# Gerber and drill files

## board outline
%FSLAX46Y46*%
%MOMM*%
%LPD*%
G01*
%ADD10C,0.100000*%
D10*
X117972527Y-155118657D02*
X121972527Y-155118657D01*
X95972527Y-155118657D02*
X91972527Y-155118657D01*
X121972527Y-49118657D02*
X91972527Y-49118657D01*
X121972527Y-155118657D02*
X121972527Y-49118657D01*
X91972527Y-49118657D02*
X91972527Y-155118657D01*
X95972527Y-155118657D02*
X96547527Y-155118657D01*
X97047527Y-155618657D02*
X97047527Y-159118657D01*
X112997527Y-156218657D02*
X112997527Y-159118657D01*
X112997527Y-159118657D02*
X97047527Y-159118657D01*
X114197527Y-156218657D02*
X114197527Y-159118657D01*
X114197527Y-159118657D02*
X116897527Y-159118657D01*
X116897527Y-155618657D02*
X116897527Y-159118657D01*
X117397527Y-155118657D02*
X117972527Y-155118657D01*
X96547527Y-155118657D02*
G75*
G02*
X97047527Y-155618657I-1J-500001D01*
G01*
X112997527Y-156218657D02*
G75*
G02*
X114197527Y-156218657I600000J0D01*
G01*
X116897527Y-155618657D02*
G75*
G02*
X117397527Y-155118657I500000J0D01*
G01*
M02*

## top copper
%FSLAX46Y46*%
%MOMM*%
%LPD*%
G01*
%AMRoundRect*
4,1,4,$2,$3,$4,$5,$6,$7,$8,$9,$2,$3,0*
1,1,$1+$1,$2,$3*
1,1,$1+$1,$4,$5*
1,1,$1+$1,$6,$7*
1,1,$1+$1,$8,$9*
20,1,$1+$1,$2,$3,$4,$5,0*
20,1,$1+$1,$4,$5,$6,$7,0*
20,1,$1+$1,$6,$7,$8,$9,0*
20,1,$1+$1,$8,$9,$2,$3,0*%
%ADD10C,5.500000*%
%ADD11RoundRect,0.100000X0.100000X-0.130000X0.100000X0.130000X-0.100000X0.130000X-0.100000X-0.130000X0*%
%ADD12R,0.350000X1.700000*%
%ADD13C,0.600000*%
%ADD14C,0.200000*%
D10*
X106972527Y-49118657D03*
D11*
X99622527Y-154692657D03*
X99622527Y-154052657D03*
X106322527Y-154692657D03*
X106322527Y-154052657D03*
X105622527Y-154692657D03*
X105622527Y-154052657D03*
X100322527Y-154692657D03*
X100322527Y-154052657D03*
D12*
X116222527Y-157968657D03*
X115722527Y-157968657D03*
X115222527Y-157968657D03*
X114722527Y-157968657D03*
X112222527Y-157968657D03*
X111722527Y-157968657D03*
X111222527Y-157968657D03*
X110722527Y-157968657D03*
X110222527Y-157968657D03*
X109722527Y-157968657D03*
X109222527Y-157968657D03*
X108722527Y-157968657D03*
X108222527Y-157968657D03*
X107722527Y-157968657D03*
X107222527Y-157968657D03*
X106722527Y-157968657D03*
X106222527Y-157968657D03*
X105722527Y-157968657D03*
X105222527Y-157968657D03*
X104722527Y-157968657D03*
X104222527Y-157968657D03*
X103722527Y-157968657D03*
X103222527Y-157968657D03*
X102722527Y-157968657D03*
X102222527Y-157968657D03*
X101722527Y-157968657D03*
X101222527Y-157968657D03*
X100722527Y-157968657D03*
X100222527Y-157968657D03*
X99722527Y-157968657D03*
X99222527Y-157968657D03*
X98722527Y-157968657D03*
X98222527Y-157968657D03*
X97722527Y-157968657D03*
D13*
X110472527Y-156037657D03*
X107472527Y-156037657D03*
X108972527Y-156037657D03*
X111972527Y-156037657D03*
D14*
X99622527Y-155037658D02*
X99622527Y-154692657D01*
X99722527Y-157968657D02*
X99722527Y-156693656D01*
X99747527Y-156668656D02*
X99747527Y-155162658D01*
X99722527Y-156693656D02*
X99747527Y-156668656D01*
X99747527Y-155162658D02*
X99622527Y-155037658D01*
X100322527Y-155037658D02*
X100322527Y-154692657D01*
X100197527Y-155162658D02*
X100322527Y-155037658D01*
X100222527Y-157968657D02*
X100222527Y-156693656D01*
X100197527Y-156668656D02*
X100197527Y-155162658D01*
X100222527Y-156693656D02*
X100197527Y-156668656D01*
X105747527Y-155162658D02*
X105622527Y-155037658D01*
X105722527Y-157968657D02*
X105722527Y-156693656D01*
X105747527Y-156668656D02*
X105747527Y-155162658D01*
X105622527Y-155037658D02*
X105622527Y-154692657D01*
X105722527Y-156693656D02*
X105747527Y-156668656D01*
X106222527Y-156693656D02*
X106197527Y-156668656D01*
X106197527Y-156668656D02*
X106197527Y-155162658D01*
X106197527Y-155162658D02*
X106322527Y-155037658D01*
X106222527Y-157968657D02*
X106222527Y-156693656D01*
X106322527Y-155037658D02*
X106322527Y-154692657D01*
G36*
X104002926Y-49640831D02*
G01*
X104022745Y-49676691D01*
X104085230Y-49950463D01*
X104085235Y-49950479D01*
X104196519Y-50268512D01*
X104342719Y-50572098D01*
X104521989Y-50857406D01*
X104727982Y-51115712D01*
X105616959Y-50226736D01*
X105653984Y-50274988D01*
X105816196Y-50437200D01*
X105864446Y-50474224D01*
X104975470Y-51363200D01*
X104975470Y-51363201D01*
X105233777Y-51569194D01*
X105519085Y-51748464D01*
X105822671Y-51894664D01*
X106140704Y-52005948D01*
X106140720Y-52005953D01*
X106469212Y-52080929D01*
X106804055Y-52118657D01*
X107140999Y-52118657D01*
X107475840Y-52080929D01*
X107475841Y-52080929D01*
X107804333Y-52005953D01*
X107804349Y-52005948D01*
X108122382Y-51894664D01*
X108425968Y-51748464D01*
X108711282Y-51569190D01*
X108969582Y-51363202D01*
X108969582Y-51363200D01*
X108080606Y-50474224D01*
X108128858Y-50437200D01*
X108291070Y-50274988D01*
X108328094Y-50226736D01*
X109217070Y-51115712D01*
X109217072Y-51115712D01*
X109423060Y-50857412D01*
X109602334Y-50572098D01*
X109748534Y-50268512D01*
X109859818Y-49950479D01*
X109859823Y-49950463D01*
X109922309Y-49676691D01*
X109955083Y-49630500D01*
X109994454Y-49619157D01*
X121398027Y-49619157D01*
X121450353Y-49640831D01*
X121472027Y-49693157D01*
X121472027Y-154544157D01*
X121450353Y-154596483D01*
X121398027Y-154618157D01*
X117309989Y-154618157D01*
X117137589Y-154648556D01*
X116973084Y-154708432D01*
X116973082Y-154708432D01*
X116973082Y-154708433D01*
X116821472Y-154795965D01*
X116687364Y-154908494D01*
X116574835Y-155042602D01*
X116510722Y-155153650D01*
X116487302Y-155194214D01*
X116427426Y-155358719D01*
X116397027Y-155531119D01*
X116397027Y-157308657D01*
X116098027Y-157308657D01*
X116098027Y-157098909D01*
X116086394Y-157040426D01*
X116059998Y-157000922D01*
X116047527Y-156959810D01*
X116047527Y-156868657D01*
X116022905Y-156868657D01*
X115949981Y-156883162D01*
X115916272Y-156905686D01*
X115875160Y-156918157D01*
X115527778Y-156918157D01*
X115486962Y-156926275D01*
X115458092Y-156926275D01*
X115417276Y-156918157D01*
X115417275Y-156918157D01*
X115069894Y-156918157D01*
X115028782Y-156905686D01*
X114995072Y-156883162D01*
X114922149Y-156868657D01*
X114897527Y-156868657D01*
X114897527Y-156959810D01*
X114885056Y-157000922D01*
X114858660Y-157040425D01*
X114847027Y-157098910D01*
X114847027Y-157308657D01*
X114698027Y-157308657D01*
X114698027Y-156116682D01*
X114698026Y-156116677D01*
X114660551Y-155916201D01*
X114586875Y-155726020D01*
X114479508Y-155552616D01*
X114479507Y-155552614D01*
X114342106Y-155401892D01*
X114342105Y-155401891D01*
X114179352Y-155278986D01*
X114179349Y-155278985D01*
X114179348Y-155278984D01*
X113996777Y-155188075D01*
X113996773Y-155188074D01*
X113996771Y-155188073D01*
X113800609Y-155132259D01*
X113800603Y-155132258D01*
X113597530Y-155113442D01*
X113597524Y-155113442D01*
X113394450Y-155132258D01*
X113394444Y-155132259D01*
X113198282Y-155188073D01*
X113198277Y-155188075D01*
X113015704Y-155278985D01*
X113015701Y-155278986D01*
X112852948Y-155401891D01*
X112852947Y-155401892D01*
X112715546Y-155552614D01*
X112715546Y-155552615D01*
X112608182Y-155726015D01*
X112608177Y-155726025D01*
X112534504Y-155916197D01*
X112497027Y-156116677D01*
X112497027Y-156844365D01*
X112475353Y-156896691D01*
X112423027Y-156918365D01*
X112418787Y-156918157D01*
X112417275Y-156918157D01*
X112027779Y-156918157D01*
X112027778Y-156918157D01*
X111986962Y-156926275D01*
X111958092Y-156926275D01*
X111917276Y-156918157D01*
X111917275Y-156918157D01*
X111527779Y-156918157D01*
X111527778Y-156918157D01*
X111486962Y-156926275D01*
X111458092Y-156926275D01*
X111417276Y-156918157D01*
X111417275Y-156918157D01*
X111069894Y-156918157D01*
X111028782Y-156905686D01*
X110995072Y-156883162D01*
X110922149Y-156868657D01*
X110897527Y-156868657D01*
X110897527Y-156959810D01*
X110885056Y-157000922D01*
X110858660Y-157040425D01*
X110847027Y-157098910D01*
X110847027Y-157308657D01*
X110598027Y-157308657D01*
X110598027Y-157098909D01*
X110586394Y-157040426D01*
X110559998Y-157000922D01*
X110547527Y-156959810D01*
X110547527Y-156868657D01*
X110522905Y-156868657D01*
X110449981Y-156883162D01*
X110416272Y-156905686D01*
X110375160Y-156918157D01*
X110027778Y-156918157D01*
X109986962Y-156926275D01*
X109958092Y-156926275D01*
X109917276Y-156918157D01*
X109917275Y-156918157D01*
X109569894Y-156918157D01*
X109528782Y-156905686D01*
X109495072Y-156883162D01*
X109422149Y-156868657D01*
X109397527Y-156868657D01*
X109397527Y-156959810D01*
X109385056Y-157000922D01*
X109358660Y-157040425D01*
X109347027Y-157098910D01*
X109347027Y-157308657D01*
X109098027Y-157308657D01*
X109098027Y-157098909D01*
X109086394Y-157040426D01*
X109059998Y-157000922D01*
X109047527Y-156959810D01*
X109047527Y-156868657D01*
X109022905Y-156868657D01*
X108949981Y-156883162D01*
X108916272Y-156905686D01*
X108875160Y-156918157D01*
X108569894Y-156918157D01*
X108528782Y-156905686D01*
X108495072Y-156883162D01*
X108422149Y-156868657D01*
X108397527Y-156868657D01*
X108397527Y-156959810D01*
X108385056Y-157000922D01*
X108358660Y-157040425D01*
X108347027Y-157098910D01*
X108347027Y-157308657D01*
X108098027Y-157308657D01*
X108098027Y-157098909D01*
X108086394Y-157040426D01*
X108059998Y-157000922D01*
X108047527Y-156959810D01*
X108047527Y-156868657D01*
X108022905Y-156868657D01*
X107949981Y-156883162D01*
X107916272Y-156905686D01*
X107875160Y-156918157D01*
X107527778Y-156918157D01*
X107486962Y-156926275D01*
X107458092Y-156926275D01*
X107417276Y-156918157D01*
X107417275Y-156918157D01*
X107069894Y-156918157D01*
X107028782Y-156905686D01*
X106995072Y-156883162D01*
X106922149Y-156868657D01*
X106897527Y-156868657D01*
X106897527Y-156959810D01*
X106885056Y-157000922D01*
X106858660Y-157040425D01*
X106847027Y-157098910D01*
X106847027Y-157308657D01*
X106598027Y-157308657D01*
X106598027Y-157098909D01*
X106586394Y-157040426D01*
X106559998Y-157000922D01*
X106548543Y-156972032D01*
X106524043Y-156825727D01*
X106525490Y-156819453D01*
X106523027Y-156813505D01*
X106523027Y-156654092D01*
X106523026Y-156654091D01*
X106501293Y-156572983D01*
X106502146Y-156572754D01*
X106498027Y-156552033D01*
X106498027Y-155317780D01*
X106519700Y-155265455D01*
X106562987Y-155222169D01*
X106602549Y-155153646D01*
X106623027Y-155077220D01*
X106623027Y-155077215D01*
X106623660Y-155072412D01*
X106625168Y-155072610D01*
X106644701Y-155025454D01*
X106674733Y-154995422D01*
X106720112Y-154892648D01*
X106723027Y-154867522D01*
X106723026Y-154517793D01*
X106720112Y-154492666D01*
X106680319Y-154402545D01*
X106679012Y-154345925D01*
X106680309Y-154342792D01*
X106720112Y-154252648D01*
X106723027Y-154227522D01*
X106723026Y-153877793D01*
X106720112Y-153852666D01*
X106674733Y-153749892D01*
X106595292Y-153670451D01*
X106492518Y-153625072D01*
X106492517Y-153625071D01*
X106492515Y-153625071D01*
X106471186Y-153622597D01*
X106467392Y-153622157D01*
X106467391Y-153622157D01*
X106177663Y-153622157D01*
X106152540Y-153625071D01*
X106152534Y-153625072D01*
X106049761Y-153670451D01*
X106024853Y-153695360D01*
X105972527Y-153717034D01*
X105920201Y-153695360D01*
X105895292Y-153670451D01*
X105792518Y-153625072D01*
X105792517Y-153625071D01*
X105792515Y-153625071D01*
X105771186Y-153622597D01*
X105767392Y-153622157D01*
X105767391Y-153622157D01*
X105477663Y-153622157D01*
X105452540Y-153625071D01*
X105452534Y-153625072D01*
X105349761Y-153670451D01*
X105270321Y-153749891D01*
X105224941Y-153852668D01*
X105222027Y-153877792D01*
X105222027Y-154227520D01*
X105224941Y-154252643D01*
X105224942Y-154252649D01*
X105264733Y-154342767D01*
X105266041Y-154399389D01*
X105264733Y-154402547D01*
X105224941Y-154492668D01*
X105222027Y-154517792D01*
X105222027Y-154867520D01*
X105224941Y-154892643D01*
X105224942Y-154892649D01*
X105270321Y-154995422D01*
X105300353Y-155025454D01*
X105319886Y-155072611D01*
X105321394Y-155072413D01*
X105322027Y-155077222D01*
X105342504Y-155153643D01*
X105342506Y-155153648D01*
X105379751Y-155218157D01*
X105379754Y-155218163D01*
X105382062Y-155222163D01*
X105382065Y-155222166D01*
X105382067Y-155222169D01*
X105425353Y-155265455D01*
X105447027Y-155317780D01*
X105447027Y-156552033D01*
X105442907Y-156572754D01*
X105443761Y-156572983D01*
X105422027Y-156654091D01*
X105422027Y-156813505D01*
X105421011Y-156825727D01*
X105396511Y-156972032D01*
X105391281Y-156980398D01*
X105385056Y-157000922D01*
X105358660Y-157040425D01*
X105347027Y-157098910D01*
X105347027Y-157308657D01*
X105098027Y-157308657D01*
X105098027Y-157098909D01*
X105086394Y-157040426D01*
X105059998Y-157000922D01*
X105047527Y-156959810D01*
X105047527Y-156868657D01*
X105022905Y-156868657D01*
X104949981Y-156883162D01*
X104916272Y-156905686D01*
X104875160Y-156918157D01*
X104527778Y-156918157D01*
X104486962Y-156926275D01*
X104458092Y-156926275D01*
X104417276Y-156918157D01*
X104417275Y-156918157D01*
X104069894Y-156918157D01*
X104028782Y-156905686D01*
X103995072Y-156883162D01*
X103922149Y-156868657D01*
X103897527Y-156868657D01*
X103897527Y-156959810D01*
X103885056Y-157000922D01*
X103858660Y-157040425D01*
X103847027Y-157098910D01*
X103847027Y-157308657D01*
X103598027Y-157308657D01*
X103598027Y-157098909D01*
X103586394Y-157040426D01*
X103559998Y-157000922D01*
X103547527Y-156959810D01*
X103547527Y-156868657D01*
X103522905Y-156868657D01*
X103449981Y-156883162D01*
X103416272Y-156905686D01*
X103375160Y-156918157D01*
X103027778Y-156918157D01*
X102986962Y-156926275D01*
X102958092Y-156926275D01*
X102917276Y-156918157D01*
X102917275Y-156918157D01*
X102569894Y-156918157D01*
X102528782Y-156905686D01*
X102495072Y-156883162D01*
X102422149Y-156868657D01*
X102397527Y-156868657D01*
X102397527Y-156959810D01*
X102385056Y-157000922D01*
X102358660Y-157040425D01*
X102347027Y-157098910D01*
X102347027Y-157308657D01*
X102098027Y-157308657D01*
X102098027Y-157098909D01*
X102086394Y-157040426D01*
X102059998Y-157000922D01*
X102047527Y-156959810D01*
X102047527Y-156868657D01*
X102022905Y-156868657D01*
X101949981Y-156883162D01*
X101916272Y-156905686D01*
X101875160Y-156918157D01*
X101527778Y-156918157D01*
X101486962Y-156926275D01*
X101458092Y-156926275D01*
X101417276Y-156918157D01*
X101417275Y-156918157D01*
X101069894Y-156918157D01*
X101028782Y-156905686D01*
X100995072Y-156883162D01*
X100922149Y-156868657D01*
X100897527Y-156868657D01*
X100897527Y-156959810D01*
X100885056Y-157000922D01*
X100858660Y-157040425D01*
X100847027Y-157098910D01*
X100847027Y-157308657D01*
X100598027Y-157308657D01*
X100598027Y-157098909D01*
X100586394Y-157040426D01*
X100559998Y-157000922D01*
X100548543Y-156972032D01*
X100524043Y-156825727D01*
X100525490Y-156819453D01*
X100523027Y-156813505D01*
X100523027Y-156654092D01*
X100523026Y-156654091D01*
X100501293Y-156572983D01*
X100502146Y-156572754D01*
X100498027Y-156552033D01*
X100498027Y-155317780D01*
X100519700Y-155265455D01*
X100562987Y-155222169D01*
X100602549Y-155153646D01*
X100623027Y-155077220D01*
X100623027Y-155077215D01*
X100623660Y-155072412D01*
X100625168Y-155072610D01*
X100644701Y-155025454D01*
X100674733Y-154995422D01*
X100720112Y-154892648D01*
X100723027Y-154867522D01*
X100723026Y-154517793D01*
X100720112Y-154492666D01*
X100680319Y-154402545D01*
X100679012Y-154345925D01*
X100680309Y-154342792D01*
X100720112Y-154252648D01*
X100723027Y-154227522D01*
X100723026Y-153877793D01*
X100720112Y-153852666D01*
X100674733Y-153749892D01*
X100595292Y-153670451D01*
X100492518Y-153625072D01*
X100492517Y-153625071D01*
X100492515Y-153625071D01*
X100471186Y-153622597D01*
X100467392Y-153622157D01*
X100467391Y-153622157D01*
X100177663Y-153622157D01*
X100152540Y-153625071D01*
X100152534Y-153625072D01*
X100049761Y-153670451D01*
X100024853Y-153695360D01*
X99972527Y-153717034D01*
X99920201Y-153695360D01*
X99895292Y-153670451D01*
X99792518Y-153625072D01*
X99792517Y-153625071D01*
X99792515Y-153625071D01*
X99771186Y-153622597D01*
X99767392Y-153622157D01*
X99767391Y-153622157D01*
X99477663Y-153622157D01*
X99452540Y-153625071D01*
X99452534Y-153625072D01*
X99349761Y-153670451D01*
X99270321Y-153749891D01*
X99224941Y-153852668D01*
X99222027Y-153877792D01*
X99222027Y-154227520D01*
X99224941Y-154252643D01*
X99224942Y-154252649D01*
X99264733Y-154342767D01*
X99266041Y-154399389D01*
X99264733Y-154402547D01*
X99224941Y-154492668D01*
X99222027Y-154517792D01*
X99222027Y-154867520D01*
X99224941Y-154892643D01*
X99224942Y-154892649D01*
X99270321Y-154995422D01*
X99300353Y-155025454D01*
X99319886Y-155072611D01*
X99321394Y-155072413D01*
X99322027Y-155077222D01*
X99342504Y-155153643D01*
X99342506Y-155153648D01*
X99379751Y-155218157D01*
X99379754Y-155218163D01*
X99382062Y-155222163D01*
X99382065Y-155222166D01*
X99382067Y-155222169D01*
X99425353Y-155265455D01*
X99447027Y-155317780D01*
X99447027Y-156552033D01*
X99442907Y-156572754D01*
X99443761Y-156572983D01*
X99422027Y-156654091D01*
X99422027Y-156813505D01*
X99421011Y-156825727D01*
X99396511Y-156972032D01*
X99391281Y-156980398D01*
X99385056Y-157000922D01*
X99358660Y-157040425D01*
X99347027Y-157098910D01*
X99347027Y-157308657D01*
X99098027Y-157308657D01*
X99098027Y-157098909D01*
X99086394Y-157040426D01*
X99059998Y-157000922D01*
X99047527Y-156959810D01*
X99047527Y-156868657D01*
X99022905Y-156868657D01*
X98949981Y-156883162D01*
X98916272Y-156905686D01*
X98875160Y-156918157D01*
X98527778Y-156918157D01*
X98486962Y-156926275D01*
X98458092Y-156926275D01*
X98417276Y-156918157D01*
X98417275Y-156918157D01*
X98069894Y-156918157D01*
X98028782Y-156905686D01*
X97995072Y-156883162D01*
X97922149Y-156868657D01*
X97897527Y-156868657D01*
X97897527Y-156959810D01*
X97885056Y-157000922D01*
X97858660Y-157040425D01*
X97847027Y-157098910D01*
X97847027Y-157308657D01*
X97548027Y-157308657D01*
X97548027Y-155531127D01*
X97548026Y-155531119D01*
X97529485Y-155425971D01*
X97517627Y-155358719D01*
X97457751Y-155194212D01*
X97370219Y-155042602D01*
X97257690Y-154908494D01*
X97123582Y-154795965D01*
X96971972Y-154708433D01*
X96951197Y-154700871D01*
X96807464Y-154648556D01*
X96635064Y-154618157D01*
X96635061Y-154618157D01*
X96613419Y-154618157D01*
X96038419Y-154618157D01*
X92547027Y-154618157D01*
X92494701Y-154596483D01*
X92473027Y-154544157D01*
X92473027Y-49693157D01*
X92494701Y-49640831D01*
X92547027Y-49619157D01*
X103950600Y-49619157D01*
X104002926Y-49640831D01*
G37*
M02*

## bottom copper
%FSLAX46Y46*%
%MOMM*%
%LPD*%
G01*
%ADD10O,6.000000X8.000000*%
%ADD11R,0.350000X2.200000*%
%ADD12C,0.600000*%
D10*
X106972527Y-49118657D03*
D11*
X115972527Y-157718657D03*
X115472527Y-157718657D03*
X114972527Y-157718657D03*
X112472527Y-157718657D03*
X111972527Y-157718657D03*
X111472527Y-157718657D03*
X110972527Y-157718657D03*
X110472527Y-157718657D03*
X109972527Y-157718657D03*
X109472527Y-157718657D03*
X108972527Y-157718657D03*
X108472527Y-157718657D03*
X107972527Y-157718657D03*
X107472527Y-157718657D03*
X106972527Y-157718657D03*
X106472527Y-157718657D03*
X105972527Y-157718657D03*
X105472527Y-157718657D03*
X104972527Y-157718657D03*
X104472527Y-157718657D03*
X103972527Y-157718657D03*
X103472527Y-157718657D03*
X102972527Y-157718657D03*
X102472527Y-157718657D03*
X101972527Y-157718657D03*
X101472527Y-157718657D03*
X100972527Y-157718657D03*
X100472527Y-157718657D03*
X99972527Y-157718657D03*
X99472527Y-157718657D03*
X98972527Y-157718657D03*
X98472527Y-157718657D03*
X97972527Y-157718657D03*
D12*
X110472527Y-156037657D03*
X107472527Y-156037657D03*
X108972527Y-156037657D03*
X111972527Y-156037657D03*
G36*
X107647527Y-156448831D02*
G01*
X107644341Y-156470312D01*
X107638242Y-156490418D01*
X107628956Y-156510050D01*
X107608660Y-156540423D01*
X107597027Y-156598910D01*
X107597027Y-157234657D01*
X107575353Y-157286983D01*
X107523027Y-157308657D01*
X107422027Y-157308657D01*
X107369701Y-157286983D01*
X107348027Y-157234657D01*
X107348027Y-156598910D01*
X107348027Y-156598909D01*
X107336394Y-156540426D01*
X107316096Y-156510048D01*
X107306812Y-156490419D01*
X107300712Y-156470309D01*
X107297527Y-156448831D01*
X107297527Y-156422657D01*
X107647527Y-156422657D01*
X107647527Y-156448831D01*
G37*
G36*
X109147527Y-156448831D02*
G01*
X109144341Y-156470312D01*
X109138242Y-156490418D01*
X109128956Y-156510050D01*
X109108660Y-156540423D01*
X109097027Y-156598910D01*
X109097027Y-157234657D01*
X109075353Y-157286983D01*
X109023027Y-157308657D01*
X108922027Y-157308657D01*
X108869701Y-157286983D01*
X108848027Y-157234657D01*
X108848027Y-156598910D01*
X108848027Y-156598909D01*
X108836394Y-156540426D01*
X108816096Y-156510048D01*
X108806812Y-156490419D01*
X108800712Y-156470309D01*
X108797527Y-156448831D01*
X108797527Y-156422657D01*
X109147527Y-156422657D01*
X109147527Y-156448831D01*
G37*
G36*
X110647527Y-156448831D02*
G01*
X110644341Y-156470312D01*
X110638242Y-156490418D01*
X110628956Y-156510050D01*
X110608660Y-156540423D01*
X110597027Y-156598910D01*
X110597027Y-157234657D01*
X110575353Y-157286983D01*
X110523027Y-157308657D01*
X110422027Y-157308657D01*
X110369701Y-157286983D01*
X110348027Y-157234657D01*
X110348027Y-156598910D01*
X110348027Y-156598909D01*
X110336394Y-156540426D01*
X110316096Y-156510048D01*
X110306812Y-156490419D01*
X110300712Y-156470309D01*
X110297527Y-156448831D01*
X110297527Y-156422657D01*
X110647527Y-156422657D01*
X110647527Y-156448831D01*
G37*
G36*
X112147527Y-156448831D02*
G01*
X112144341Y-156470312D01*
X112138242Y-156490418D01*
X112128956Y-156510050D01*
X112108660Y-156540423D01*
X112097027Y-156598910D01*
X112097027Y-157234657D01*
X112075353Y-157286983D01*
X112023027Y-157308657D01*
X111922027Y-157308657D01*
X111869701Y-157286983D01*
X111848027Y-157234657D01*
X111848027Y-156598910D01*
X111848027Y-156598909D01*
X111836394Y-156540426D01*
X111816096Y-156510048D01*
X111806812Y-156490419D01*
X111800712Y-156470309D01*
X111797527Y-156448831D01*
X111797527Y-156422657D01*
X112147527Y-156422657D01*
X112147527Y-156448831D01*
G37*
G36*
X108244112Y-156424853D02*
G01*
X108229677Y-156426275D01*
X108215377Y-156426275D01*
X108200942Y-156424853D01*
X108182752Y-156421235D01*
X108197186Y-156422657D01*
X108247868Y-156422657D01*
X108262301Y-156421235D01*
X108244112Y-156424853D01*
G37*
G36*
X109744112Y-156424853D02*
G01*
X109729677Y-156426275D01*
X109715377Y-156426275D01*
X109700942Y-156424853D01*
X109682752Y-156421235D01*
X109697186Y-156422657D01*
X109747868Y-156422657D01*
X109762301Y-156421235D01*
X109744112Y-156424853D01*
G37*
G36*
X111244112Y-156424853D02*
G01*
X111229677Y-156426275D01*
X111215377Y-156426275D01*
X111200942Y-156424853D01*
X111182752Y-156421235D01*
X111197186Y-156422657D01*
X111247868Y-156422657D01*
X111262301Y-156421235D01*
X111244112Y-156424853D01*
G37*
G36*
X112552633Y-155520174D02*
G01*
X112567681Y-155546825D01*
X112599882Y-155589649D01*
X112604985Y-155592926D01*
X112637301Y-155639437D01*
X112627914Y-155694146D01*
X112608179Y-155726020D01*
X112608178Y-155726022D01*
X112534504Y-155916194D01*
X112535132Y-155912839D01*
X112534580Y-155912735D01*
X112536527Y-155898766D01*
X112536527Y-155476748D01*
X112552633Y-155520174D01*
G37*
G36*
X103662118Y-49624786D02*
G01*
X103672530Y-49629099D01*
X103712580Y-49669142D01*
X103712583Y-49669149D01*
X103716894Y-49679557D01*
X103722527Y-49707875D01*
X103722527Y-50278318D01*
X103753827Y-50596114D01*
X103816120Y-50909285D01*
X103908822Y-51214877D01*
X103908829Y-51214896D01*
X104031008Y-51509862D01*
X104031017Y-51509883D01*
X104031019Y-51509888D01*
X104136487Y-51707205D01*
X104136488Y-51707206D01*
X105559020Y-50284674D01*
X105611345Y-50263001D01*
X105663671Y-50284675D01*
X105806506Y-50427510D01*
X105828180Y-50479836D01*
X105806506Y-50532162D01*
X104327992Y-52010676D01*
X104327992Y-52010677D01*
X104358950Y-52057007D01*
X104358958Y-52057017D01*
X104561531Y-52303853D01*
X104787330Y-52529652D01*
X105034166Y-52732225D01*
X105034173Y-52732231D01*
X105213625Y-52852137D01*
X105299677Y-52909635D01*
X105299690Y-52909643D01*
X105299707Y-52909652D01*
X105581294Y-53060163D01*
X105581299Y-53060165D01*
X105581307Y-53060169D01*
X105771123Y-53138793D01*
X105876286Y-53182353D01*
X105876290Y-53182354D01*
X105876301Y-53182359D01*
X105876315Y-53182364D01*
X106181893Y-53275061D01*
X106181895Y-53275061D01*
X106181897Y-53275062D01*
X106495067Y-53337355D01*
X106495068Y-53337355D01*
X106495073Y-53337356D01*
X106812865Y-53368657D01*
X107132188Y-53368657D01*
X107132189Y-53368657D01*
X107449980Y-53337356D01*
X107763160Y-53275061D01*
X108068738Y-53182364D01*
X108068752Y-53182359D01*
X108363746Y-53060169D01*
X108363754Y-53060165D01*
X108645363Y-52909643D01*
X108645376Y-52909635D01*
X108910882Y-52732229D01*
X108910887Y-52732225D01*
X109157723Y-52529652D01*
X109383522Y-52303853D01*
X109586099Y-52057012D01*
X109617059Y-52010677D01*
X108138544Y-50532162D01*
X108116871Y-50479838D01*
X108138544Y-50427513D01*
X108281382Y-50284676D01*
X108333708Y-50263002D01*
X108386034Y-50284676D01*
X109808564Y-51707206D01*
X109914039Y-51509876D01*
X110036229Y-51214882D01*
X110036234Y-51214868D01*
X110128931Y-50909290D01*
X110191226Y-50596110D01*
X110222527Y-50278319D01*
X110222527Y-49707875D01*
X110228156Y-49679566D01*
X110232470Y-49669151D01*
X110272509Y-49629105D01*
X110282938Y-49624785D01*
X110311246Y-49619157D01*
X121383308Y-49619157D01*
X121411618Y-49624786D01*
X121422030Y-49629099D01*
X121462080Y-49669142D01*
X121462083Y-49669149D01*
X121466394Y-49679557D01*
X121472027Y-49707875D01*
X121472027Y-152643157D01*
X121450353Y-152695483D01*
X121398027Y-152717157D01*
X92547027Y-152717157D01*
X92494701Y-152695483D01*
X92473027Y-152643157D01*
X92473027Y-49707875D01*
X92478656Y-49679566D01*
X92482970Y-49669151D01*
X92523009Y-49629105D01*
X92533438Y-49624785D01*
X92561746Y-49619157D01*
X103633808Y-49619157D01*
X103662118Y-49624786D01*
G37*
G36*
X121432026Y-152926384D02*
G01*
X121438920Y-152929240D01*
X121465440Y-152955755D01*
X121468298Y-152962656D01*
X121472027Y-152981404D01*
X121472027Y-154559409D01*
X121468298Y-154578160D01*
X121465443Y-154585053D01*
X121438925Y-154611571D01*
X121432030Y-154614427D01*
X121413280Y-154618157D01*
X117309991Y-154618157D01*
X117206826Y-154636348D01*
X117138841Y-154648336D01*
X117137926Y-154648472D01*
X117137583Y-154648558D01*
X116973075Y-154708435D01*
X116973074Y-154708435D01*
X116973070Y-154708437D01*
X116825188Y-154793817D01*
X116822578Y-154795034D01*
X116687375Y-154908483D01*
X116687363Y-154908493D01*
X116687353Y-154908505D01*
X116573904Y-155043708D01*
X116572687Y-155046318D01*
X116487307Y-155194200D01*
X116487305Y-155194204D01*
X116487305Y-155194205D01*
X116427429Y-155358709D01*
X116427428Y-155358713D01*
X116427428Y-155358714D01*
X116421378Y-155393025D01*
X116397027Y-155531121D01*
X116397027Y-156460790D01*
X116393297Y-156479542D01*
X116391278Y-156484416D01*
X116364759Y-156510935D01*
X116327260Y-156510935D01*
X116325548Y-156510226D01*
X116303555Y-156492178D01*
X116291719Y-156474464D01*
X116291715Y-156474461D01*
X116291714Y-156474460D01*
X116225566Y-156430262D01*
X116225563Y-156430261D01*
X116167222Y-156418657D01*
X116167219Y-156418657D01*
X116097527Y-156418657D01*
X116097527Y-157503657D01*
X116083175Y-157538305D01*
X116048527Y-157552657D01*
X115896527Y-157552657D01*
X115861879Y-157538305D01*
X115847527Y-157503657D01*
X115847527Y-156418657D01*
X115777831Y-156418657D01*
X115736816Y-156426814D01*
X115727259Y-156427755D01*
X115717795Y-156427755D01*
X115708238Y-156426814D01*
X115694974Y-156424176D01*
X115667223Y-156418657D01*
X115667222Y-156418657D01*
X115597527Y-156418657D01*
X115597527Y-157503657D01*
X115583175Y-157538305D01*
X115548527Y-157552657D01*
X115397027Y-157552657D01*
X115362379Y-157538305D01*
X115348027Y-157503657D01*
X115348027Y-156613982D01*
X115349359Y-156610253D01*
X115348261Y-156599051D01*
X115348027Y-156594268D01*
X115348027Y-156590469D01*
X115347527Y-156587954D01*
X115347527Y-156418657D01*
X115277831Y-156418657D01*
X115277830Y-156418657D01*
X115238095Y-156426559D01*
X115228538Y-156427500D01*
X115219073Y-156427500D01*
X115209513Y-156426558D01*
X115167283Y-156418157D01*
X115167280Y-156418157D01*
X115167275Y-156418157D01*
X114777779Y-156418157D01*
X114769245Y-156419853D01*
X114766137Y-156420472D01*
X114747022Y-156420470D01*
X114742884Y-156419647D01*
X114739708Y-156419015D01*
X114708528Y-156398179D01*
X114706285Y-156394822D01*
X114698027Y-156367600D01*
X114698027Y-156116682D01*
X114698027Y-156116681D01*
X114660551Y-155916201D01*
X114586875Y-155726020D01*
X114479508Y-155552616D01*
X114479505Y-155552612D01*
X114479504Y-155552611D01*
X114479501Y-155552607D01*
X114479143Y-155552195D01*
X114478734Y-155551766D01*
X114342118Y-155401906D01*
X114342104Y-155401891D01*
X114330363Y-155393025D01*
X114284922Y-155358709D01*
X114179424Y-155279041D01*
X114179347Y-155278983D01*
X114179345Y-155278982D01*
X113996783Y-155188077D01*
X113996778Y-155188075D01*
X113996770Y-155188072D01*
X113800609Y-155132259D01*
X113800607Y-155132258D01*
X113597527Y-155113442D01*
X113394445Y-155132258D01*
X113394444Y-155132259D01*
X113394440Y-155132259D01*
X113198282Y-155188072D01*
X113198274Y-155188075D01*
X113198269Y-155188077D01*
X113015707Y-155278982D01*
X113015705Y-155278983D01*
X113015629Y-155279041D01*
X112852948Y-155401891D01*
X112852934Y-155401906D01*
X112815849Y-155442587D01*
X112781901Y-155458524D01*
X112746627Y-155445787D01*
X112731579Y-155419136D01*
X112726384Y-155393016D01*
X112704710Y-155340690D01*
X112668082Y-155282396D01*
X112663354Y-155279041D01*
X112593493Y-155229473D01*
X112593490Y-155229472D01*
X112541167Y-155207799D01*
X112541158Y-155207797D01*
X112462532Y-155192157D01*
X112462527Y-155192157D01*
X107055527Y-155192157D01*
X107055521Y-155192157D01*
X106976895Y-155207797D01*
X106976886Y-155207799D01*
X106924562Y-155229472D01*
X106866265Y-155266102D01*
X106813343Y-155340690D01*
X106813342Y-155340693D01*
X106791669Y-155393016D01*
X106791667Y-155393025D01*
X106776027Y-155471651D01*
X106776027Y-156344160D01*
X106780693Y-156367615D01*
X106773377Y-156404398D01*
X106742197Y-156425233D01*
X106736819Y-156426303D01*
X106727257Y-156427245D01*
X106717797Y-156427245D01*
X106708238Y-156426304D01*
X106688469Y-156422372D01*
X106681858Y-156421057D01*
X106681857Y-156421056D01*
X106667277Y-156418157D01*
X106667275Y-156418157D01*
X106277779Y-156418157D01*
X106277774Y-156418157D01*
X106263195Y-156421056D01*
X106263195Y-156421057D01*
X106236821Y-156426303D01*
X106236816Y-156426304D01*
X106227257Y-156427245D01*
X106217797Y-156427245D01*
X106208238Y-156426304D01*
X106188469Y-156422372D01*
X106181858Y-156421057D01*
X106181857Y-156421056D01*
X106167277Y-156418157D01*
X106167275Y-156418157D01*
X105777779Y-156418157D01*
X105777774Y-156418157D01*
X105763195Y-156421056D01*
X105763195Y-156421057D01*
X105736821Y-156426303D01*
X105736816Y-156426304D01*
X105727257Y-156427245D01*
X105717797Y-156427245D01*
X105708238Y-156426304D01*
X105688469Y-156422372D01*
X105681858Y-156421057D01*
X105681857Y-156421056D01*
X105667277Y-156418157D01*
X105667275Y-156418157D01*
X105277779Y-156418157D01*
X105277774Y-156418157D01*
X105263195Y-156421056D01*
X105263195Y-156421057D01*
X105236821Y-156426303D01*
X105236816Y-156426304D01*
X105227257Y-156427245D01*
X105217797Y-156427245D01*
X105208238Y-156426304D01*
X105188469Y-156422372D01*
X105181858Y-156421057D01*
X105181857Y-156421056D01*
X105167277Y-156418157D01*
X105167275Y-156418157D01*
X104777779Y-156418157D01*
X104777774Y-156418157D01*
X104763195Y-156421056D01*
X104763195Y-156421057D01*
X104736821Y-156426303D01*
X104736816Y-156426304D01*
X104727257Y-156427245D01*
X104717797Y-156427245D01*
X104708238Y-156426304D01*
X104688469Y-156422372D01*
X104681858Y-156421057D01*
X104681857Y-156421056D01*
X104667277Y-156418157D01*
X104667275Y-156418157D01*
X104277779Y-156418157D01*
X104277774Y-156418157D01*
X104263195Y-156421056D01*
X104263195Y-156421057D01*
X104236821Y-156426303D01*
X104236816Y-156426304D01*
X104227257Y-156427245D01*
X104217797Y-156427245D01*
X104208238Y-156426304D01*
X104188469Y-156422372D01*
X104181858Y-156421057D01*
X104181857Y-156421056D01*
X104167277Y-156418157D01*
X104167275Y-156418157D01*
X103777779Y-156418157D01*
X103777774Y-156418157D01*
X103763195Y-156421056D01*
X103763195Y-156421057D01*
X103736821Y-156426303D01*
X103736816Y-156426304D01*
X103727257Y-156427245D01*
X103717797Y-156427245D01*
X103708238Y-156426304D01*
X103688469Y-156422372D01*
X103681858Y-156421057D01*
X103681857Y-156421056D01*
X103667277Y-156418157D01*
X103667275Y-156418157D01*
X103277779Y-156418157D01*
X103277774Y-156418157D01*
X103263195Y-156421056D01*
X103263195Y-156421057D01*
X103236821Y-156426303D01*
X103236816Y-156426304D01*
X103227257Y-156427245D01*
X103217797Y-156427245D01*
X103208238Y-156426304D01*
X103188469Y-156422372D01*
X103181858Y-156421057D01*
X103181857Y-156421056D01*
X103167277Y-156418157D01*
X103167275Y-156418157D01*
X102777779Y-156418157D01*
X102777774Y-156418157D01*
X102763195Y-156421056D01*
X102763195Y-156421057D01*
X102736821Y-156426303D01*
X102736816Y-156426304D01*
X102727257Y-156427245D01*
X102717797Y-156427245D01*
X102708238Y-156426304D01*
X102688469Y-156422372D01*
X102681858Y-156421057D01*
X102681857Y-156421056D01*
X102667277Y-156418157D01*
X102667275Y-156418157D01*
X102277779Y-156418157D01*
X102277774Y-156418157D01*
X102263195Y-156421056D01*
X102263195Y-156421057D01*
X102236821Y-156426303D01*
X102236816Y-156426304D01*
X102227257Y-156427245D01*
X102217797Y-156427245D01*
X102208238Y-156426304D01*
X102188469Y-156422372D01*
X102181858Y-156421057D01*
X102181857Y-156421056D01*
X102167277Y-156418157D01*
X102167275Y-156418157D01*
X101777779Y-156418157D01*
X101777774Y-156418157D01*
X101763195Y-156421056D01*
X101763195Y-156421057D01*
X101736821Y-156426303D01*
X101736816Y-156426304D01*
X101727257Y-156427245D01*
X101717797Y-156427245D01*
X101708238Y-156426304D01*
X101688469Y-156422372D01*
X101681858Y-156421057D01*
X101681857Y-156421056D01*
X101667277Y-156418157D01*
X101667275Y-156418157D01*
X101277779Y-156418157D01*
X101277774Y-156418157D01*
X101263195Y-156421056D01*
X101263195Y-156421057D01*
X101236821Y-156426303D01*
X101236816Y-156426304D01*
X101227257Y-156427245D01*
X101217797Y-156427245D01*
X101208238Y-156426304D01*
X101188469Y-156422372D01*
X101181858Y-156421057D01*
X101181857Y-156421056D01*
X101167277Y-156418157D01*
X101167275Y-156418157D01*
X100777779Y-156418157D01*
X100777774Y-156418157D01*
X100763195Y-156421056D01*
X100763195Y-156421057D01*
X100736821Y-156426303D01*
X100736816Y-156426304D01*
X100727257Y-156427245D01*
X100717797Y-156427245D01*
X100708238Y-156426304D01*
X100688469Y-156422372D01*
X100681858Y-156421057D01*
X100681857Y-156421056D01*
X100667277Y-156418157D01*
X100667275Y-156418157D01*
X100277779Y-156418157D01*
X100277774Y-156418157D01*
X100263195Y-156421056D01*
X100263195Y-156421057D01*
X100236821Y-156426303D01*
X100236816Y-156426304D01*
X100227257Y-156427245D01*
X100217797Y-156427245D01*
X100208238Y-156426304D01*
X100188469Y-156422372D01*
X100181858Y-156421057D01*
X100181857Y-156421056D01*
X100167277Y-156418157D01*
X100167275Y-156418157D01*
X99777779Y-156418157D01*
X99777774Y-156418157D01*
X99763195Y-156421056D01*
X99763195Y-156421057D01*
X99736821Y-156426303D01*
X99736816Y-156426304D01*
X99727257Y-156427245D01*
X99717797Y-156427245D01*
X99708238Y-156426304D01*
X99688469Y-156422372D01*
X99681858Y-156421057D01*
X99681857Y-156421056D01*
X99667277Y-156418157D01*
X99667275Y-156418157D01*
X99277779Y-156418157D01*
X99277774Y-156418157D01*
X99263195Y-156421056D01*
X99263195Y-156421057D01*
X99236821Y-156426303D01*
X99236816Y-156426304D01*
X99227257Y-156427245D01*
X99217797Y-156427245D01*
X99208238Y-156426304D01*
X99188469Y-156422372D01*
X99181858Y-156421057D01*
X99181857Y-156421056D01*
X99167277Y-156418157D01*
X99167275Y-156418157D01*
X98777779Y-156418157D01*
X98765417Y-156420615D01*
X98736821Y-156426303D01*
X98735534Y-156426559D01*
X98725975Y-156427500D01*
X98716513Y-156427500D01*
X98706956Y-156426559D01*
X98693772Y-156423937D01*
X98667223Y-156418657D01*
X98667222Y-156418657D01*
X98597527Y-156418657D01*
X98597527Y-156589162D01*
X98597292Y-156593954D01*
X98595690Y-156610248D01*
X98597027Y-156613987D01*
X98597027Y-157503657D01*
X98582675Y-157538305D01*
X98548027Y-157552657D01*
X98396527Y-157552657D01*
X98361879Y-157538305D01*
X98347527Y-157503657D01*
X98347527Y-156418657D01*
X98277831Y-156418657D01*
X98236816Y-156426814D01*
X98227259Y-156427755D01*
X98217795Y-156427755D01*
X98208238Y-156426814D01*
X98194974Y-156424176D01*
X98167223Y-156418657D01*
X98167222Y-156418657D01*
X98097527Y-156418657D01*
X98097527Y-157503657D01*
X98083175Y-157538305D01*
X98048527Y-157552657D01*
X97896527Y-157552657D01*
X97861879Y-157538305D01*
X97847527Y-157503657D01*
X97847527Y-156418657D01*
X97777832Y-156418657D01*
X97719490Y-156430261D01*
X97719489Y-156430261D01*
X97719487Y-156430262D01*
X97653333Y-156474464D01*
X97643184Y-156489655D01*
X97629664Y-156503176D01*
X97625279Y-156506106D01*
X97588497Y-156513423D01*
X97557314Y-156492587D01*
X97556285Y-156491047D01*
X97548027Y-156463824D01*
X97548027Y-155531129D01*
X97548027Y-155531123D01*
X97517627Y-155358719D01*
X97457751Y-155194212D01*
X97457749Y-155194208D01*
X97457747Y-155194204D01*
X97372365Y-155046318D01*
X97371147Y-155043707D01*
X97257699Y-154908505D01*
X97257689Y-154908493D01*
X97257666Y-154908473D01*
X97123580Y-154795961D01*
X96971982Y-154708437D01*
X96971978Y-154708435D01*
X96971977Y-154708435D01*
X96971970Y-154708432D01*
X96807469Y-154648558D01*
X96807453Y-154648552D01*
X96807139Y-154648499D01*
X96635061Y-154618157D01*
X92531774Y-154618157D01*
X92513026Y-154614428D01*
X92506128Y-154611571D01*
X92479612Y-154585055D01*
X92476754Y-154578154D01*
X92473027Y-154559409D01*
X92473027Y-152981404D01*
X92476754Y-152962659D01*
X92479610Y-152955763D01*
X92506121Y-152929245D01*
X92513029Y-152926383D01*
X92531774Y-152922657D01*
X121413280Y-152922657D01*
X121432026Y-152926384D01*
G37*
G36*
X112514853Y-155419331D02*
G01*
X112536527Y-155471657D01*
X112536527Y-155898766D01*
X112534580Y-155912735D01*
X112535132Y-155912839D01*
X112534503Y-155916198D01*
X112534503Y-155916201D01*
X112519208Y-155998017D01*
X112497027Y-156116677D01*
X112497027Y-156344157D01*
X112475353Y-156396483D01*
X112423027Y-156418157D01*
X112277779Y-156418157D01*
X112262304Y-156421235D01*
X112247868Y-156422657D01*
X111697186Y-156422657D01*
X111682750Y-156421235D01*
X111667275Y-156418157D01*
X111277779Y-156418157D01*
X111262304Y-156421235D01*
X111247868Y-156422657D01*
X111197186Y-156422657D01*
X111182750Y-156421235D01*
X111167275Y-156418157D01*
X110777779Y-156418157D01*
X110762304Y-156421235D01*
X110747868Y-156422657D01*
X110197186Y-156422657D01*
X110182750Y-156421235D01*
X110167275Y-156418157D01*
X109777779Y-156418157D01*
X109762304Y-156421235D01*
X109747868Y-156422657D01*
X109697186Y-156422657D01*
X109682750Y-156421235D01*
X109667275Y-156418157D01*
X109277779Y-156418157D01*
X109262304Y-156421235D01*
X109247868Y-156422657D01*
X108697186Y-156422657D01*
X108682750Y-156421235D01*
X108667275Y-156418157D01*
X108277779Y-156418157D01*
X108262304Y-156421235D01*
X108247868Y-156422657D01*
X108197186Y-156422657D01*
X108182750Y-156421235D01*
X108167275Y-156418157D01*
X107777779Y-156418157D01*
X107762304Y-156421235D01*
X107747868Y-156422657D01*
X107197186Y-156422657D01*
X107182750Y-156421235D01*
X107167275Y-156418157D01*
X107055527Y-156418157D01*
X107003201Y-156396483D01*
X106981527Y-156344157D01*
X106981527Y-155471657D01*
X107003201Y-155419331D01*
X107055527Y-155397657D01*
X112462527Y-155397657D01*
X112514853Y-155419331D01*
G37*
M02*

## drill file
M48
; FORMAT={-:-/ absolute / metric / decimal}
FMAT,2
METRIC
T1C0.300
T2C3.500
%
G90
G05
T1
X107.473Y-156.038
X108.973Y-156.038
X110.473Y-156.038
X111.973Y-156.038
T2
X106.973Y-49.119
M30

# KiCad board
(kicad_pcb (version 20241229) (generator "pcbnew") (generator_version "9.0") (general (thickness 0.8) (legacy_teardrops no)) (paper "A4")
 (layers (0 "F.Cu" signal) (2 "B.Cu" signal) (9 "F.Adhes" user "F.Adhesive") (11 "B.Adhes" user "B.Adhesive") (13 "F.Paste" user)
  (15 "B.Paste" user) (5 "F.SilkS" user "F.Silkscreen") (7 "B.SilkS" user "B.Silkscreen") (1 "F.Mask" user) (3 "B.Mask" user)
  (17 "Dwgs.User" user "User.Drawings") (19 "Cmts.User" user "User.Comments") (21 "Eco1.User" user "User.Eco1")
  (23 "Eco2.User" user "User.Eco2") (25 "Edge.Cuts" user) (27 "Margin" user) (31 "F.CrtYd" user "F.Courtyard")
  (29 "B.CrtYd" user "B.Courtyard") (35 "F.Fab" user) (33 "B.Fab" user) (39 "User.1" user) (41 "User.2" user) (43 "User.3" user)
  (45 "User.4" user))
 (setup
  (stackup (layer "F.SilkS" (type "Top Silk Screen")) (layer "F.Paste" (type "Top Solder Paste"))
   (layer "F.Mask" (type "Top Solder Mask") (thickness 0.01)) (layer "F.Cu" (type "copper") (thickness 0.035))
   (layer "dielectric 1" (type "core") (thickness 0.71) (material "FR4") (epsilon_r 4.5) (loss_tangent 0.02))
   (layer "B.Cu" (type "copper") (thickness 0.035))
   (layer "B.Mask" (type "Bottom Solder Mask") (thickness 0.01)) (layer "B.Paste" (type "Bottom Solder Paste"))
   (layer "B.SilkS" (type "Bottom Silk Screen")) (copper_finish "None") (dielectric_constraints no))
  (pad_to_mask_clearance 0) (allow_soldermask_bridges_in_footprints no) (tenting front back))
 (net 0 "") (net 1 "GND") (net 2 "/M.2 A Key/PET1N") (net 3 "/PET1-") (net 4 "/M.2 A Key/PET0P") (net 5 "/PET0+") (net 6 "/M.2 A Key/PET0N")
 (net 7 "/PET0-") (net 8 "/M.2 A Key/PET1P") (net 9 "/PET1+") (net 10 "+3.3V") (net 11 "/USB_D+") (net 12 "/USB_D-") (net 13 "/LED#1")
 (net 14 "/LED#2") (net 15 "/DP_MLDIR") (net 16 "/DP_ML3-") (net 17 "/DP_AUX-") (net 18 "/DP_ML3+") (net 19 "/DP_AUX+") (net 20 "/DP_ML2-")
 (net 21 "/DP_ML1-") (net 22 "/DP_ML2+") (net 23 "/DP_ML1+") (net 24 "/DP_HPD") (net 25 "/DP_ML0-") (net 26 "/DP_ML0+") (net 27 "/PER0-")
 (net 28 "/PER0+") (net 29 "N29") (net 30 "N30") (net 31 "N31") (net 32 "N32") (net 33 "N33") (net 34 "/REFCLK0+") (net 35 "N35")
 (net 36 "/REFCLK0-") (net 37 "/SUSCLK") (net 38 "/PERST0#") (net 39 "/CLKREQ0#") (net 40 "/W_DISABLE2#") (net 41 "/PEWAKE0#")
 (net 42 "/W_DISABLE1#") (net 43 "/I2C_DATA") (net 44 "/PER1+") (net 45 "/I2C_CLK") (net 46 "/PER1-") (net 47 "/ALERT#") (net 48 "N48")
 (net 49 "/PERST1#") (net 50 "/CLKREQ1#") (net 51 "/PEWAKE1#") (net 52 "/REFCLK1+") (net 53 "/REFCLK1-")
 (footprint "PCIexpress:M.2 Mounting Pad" (layer "F.Cu") (at 106.972527 49.118657)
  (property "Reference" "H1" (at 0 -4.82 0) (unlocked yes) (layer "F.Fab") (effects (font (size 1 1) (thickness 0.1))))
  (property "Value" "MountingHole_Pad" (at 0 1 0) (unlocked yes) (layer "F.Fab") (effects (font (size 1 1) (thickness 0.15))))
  (pad "1" thru_hole circle (at 0 0) (size 5.5 5.5) (drill 3.5) (layers "*.Cu" "*.Mask") (remove_unused_layers no) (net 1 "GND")
   (padstack (mode front_inner_back)
    (layer "Inner" (shape circle) (size 5.5 5.5) (zone_connect -1))
    (layer "B.Cu" (shape oval) (size 6 8) (thermal_bridge_angle 45) (zone_connect -1)))))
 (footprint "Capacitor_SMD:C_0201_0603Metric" (layer "F.Cu") (at 99.622527 154.372657 90)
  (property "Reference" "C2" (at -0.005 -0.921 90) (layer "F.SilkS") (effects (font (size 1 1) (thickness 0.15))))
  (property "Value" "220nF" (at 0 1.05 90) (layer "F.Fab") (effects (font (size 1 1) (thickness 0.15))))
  (pad "" smd roundrect (at -0.345 0 90) (size 0.318 0.36) (layers "F.Paste") (roundrect_rratio 0.25))
  (pad "" smd roundrect (at 0.345 0 90) (size 0.318 0.36) (layers "F.Paste") (roundrect_rratio 0.25))
  (pad "1" smd roundrect (at -0.32 0 90) (size 0.46 0.4) (layers "F.Cu" "F.Mask") (roundrect_rratio 0.25) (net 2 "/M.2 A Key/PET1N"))
  (pad "2" smd roundrect (at 0.32 0 90) (size 0.46 0.4) (layers "F.Cu" "F.Mask") (roundrect_rratio 0.25) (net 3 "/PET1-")))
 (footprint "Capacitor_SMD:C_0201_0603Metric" (layer "F.Cu") (at 106.322527 154.372657 90)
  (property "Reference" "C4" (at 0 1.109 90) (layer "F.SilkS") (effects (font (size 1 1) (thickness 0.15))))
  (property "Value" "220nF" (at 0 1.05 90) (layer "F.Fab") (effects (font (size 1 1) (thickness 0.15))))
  (pad "" smd roundrect (at -0.345 0 90) (size 0.318 0.36) (layers "F.Paste") (roundrect_rratio 0.25))
  (pad "" smd roundrect (at 0.345 0 90) (size 0.318 0.36) (layers "F.Paste") (roundrect_rratio 0.25))
  (pad "1" smd roundrect (at -0.32 0 90) (size 0.46 0.4) (layers "F.Cu" "F.Mask") (roundrect_rratio 0.25) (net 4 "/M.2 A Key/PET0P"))
  (pad "2" smd roundrect (at 0.32 0 90) (size 0.46 0.4) (layers "F.Cu" "F.Mask") (roundrect_rratio 0.25) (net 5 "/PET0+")))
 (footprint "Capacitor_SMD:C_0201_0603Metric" (layer "F.Cu") (at 105.622527 154.372657 90)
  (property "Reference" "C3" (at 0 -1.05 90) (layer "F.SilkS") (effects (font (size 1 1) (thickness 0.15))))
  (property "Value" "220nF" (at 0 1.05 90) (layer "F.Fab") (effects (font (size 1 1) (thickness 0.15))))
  (pad "" smd roundrect (at -0.345 0 90) (size 0.318 0.36) (layers "F.Paste") (roundrect_rratio 0.25))
  (pad "" smd roundrect (at 0.345 0 90) (size 0.318 0.36) (layers "F.Paste") (roundrect_rratio 0.25))
  (pad "1" smd roundrect (at -0.32 0 90) (size 0.46 0.4) (layers "F.Cu" "F.Mask") (roundrect_rratio 0.25) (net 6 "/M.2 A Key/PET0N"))
  (pad "2" smd roundrect (at 0.32 0 90) (size 0.46 0.4) (layers "F.Cu" "F.Mask") (roundrect_rratio 0.25) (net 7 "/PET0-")))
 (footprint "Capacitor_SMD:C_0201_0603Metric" (layer "F.Cu") (at 100.322527 154.372657 90)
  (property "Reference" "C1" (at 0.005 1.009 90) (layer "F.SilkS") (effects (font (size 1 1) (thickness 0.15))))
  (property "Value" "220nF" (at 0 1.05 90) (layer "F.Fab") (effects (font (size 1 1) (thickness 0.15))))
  (pad "" smd roundrect (at -0.345 0 90) (size 0.318 0.36) (layers "F.Paste") (roundrect_rratio 0.25))
  (pad "" smd roundrect (at 0.345 0 90) (size 0.318 0.36) (layers "F.Paste") (roundrect_rratio 0.25))
  (pad "1" smd roundrect (at -0.32 0 90) (size 0.46 0.4) (layers "F.Cu" "F.Mask") (roundrect_rratio 0.25) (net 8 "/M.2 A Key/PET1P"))
  (pad "2" smd roundrect (at 0.32 0 90) (size 0.46 0.4) (layers "F.Cu" "F.Mask") (roundrect_rratio 0.25) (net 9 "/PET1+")))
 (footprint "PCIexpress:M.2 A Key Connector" (layer "F.Cu") (at 106.972527 158.008657)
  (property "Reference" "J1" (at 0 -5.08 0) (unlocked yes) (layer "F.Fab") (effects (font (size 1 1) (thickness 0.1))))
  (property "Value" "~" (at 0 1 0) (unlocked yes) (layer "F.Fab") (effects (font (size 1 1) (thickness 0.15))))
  (fp_line (start -11 -2.89) (end -10.425 -2.89) (stroke (width 0.1) (type default)) (layer "Edge.Cuts"))
  (fp_line (start -9.925 -2.39) (end -9.925 1.11) (stroke (width 0.1) (type default)) (layer "Edge.Cuts"))
  (fp_line (start 6.025 -1.79) (end 6.025 1.11) (stroke (width 0.1) (type default)) (layer "Edge.Cuts"))
  (fp_line (start 6.025 1.11) (end -9.925 1.11) (stroke (width 0.1) (type default)) (layer "Edge.Cuts"))
  (fp_line (start 7.225 -1.79) (end 7.225 1.11) (stroke (width 0.1) (type default)) (layer "Edge.Cuts"))
  (fp_line (start 7.225 1.11) (end 9.925 1.11) (stroke (width 0.1) (type default)) (layer "Edge.Cuts"))
  (fp_line (start 9.925 -2.39) (end 9.925 1.11) (stroke (width 0.1) (type default)) (layer "Edge.Cuts"))
  (fp_line (start 10.425 -2.89) (end 11 -2.89) (stroke (width 0.1) (type default)) (layer "Edge.Cuts"))
  (fp_arc (start -10.425 -2.89) (mid -10.071447 -2.743553) (end -9.925 -2.39) (stroke (width 0.1) (type default)) (layer "Edge.Cuts"))
  (fp_arc (start 6.025 -1.79) (mid 6.625 -2.39) (end 7.225 -1.79) (stroke (width 0.1) (type default)) (layer "Edge.Cuts"))
  (fp_arc (start 9.925 -2.39) (mid 10.071447 -2.743553) (end 10.425 -2.89) (stroke (width 0.1) (type default)) (layer "Edge.Cuts"))
  (pad "1" smd rect (at 9.25 -0.04 180) (size 0.35 1.7) (layers "F.Cu") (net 1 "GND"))
  (pad "2" smd rect (at 9 -0.29 180) (size 0.35 2.2) (layers "B.Cu") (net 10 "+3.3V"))
  (pad "3" smd rect (at 8.75 -0.04 180) (size 0.35 1.7) (layers "F.Cu") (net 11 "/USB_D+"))
  (pad "4" smd rect (at 8.5 -0.29 180) (size 0.35 2.2) (layers "B.Cu") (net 10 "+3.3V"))
  (pad "5" smd rect (at 8.25 -0.04 180) (size 0.35 1.7) (layers "F.Cu") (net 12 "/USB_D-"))
  (pad "6" smd rect (at 8 -0.29 180) (size 0.35 2.2) (layers "B.Cu") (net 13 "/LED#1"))
  (pad "7" smd rect (at 7.75 -0.04 180) (size 0.35 1.7) (layers "F.Cu") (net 1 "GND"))
  (pad "16" smd rect (at 5.5 -0.29 180) (size 0.35 2.2) (layers "B.Cu") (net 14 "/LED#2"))
  (pad "17" smd rect (at 5.25 -0.04 180) (size 0.35 1.7) (layers "F.Cu") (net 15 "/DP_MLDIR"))
  (pad "18" smd rect (at 5 -0.29 180) (size 0.35 2.2) (layers "B.Cu") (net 1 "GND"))
  (pad "19" smd rect (at 4.75 -0.04 180) (size 0.35 1.7) (layers "F.Cu") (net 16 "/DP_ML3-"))
  (pad "20" smd rect (at 4.5 -0.29 180) (size 0.35 2.2) (layers "B.Cu") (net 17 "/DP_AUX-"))
  (pad "21" smd rect (at 4.25 -0.04 180) (size 0.35 1.7) (layers "F.Cu") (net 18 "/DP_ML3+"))
  (pad "22" smd rect (at 4 -0.29 180) (size 0.35 2.2) (layers "B.Cu") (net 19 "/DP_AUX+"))
  (pad "23" smd rect (at 3.75 -0.04 180) (size 0.35 1.7) (layers "F.Cu") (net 1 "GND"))
  (pad "24" smd rect (at 3.5 -0.29 180) (size 0.35 2.2) (layers "B.Cu") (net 1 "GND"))
  (pad "25" smd rect (at 3.25 -0.04 180) (size 0.35 1.7) (layers "F.Cu") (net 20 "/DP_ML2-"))
  (pad "26" smd rect (at 3 -0.29 180) (size 0.35 2.2) (layers "B.Cu") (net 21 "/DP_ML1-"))
  (pad "27" smd rect (at 2.75 -0.04 180) (size 0.35 1.7) (layers "F.Cu") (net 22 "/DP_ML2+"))
  (pad "28" smd rect (at 2.5 -0.29 180) (size 0.35 2.2) (layers "B.Cu") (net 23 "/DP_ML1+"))
  (pad "29" smd rect (at 2.25 -0.04 180) (size 0.35 1.7) (layers "F.Cu") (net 1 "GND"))
  (pad "30" smd rect (at 2 -0.29 180) (size 0.35 2.2) (layers "B.Cu") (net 1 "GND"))
  (pad "31" smd rect (at 1.75 -0.04 180) (size 0.35 1.7) (layers "F.Cu") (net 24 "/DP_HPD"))
  (pad "32" smd rect (at 1.5 -0.29 180) (size 0.35 2.2) (layers "B.Cu") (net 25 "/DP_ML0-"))
  (pad "33" smd rect (at 1.25 -0.04 180) (size 0.35 1.7) (layers "F.Cu") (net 1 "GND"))
  (pad "34" smd rect (at 1 -0.29 180) (size 0.35 2.2) (layers "B.Cu") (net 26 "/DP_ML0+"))
  (pad "35" smd rect (at 0.75 -0.04 180) (size 0.35 1.7) (layers "F.Cu") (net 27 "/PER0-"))
  (pad "36" smd rect (at 0.5 -0.29 180) (size 0.35 2.2) (layers "B.Cu") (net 1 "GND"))
  (pad "37" smd rect (at 0.25 -0.04 180) (size 0.35 1.7) (layers "F.Cu") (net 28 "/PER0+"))
  (pad "38" smd rect (at 0 -0.29 180) (size 0.35 2.2) (layers "B.Cu") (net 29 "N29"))
  (pad "39" smd rect (at -0.25 -0.04 180) (size 0.35 1.7) (layers "F.Cu") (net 1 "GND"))
  (pad "40" smd rect (at -0.5 -0.29 180) (size 0.35 2.2) (layers "B.Cu") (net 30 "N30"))
  (pad "41" smd rect (at -0.75 -0.04 180) (size 0.35 1.7) (layers "F.Cu") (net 4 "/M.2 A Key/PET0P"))
  (pad "42" smd rect (at -1 -0.29 180) (size 0.35 2.2) (layers "B.Cu") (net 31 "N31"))
  (pad "43" smd rect (at -1.25 -0.04 180) (size 0.35 1.7) (layers "F.Cu") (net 6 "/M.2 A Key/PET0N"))
  (pad "44" smd rect (at -1.5 -0.29 180) (size 0.35 2.2) (layers "B.Cu") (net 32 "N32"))
  (pad "45" smd rect (at -1.75 -0.04 180) (size 0.35 1.7) (layers "F.Cu") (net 1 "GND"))
  (pad "46" smd rect (at -2 -0.29 180) (size 0.35 2.2) (layers "B.Cu") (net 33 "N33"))
  (pad "47" smd rect (at -2.25 -0.04 180) (size 0.35 1.7) (layers "F.Cu") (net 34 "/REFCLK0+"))
  (pad "48" smd rect (at -2.5 -0.29 180) (size 0.35 2.2) (layers "B.Cu") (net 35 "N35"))
  (pad "49" smd rect (at -2.75 -0.04 180) (size 0.35 1.7) (layers "F.Cu") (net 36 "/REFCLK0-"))
  (pad "50" smd rect (at -3 -0.29 180) (size 0.35 2.2) (layers "B.Cu") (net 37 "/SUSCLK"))
  (pad "51" smd rect (at -3.25 -0.04 180) (size 0.35 1.7) (layers "F.Cu") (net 1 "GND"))
  (pad "52" smd rect (at -3.5 -0.29 180) (size 0.35 2.2) (layers "B.Cu") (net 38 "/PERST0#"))
  (pad "53" smd rect (at -3.75 -0.04 180) (size 0.35 1.7) (layers "F.Cu") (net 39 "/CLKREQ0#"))
  (pad "54" smd rect (at -4 -0.29 180) (size 0.35 2.2) (layers "B.Cu") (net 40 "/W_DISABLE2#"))
  (pad "55" smd rect (at -4.25 -0.04 180) (size 0.35 1.7) (layers "F.Cu") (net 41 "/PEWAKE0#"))
  (pad "56" smd rect (at -4.5 -0.29 180) (size 0.35 2.2) (layers "B.Cu") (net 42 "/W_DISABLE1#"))
  (pad "57" smd rect (at -4.75 -0.04 180) (size 0.35 1.7) (layers "F.Cu") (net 1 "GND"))
  (pad "58" smd rect (at -5 -0.29 180) (size 0.35 2.2) (layers "B.Cu") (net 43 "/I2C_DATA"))
  (pad "59" smd rect (at -5.25 -0.04 180) (size 0.35 1.7) (layers "F.Cu") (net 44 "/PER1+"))
  (pad "60" smd rect (at -5.5 -0.29 180) (size 0.35 2.2) (layers "B.Cu") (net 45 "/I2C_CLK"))
  (pad "61" smd rect (at -5.75 -0.04 180) (size 0.35 1.7) (layers "F.Cu") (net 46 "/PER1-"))
  (pad "62" smd rect (at -6 -0.29 180) (size 0.35 2.2) (layers "B.Cu") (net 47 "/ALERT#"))
  (pad "63" smd rect (at -6.25 -0.04 180) (size 0.35 1.7) (layers "F.Cu") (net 1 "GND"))
  (pad "64" smd rect (at -6.5 -0.29 180) (size 0.35 2.2) (layers "B.Cu") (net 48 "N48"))
  (pad "65" smd rect (at -6.75 -0.04 180) (size 0.35 1.7) (layers "F.Cu") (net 8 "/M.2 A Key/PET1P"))
  (pad "66" smd rect (at -7 -0.29 180) (size 0.35 2.2) (layers "B.Cu") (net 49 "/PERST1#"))
  (pad "67" smd rect (at -7.25 -0.04 180) (size 0.35 1.7) (layers "F.Cu") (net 2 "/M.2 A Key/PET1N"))
  (pad "68" smd rect (at -7.5 -0.29 180) (size 0.35 2.2) (layers "B.Cu") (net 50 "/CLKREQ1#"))
  (pad "69" smd rect (at -7.75 -0.04 180) (size 0.35 1.7) (layers "F.Cu") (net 1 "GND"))
  (pad "70" smd rect (at -8 -0.29 180) (size 0.35 2.2) (layers "B.Cu") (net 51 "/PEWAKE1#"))
  (pad "71" smd rect (at -8.25 -0.04 180) (size 0.35 1.7) (layers "F.Cu") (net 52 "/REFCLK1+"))
  (pad "72" smd rect (at -8.5 -0.29 180) (size 0.35 2.2) (layers "B.Cu") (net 10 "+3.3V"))
  (pad "73" smd rect (at -8.75 -0.04 180) (size 0.35 1.7) (layers "F.Cu") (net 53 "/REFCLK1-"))
  (pad "74" smd rect (at -9 -0.29 180) (size 0.35 2.2) (layers "B.Cu") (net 10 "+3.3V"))
  (pad "75" smd rect (at -9.25 -0.04 180) (size 0.35 1.7) (layers "F.Cu") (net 1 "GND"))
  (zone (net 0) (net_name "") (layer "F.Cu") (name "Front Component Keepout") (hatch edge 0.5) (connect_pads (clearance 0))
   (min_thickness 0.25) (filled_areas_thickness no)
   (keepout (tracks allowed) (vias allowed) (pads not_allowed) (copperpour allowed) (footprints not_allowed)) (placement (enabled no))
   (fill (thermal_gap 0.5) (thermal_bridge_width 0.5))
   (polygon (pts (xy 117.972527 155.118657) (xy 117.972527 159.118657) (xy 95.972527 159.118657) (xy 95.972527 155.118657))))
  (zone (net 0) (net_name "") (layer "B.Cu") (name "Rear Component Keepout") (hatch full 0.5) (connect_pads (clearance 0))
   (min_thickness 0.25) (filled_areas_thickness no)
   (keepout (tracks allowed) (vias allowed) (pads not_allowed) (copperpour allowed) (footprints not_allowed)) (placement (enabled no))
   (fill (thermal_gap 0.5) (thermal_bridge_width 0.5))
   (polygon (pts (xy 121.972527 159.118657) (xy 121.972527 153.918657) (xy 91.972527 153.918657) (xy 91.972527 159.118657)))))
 (gr_line (start 117.972527 155.118657) (end 121.972527 155.118657) (stroke (width 0.1) (type default)) (layer "Edge.Cuts"))
 (gr_line (start 95.972527 155.118657) (end 91.972527 155.118657) (stroke (width 0.1) (type default)) (layer "Edge.Cuts"))
 (gr_line (start 121.972527 49.118657) (end 91.972527 49.118657) (stroke (width 0.1) (type solid)) (layer "Edge.Cuts"))
 (gr_line (start 121.972527 155.118657) (end 121.972527 49.118657) (stroke (width 0.1) (type default)) (layer "Edge.Cuts"))
 (gr_line (start 91.972527 49.118657) (end 91.972527 155.118657) (stroke (width 0.1) (type default)) (layer "Edge.Cuts"))
 (via (at 110.472527 156.037657) (size 0.6) (drill 0.3) (layers "F.Cu" "B.Cu") (free yes) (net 1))
 (via (at 107.472527 156.037657) (size 0.6) (drill 0.3) (layers "F.Cu" "B.Cu") (free yes) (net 1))
 (via (at 108.972527 156.037657) (size 0.6) (drill 0.3) (layers "F.Cu" "B.Cu") (free yes) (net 1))
 (via (at 111.972527 156.037657) (size 0.6) (drill 0.3) (layers "F.Cu" "B.Cu") (free yes) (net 1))
 (segment (start 99.622527 155.037658) (end 99.622527 154.692657) (width 0.2) (layer "F.Cu") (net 2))
 (segment (start 99.722527 157.968657) (end 99.722527 156.693656) (width 0.2) (layer "F.Cu") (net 2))
 (segment (start 99.747527 156.668656) (end 99.747527 155.162658) (width 0.2) (layer "F.Cu") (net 2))
 (segment (start 99.722527 156.693656) (end 99.747527 156.668656) (width 0.2) (layer "F.Cu") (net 2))
 (segment (start 99.747527 155.162658) (end 99.622527 155.037658) (width 0.2) (layer "F.Cu") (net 2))
 (segment (start 100.322527 155.037658) (end 100.322527 154.692657) (width 0.2) (layer "F.Cu") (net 8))
 (segment (start 100.197527 155.162658) (end 100.322527 155.037658) (width 0.2) (layer "F.Cu") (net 8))
 (segment (start 100.222527 157.968657) (end 100.222527 156.693656) (width 0.2) (layer "F.Cu") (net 8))
 (segment (start 100.197527 156.668656) (end 100.197527 155.162658) (width 0.2) (layer "F.Cu") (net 8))
 (segment (start 100.222527 156.693656) (end 100.197527 156.668656) (width 0.2) (layer "F.Cu") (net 8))
 (segment (start 105.747527 155.162658) (end 105.622527 155.037658) (width 0.2) (layer "F.Cu") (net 6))
 (segment (start 105.722527 157.968657) (end 105.722527 156.693656) (width 0.2) (layer "F.Cu") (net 6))
 (segment (start 105.747527 156.668656) (end 105.747527 155.162658) (width 0.2) (layer "F.Cu") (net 6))
 (segment (start 105.622527 155.037658) (end 105.622527 154.692657) (width 0.2) (layer "F.Cu") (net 6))
 (segment (start 105.722527 156.693656) (end 105.747527 156.668656) (width 0.2) (layer "F.Cu") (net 6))
 (segment (start 106.222527 156.693656) (end 106.197527 156.668656) (width 0.2) (layer "F.Cu") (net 4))
 (segment (start 106.197527 156.668656) (end 106.197527 155.162658) (width 0.2) (layer "F.Cu") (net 4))
 (segment (start 106.197527 155.162658) (end 106.322527 155.037658) (width 0.2) (layer "F.Cu") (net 4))
 (segment (start 106.222527 157.968657) (end 106.222527 156.693656) (width 0.2) (layer "F.Cu") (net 4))
 (segment (start 106.322527 155.037658) (end 106.322527 154.692657) (width 0.2) (layer "F.Cu") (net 4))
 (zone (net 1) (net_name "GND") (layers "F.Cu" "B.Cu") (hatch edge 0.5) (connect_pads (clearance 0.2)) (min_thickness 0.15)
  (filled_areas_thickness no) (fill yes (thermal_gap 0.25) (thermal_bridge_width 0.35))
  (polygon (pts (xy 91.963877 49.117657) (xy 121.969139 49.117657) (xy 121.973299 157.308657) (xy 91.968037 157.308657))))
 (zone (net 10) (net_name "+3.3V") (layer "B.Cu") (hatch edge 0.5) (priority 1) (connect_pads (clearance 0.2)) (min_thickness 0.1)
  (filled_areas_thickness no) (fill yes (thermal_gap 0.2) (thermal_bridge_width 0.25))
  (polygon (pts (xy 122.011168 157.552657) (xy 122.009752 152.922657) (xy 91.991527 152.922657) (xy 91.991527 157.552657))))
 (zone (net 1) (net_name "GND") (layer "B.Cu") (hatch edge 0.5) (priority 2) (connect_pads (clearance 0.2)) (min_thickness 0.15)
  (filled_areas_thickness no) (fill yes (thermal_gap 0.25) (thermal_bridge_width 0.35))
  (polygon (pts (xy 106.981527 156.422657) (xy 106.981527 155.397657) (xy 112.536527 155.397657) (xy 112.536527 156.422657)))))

